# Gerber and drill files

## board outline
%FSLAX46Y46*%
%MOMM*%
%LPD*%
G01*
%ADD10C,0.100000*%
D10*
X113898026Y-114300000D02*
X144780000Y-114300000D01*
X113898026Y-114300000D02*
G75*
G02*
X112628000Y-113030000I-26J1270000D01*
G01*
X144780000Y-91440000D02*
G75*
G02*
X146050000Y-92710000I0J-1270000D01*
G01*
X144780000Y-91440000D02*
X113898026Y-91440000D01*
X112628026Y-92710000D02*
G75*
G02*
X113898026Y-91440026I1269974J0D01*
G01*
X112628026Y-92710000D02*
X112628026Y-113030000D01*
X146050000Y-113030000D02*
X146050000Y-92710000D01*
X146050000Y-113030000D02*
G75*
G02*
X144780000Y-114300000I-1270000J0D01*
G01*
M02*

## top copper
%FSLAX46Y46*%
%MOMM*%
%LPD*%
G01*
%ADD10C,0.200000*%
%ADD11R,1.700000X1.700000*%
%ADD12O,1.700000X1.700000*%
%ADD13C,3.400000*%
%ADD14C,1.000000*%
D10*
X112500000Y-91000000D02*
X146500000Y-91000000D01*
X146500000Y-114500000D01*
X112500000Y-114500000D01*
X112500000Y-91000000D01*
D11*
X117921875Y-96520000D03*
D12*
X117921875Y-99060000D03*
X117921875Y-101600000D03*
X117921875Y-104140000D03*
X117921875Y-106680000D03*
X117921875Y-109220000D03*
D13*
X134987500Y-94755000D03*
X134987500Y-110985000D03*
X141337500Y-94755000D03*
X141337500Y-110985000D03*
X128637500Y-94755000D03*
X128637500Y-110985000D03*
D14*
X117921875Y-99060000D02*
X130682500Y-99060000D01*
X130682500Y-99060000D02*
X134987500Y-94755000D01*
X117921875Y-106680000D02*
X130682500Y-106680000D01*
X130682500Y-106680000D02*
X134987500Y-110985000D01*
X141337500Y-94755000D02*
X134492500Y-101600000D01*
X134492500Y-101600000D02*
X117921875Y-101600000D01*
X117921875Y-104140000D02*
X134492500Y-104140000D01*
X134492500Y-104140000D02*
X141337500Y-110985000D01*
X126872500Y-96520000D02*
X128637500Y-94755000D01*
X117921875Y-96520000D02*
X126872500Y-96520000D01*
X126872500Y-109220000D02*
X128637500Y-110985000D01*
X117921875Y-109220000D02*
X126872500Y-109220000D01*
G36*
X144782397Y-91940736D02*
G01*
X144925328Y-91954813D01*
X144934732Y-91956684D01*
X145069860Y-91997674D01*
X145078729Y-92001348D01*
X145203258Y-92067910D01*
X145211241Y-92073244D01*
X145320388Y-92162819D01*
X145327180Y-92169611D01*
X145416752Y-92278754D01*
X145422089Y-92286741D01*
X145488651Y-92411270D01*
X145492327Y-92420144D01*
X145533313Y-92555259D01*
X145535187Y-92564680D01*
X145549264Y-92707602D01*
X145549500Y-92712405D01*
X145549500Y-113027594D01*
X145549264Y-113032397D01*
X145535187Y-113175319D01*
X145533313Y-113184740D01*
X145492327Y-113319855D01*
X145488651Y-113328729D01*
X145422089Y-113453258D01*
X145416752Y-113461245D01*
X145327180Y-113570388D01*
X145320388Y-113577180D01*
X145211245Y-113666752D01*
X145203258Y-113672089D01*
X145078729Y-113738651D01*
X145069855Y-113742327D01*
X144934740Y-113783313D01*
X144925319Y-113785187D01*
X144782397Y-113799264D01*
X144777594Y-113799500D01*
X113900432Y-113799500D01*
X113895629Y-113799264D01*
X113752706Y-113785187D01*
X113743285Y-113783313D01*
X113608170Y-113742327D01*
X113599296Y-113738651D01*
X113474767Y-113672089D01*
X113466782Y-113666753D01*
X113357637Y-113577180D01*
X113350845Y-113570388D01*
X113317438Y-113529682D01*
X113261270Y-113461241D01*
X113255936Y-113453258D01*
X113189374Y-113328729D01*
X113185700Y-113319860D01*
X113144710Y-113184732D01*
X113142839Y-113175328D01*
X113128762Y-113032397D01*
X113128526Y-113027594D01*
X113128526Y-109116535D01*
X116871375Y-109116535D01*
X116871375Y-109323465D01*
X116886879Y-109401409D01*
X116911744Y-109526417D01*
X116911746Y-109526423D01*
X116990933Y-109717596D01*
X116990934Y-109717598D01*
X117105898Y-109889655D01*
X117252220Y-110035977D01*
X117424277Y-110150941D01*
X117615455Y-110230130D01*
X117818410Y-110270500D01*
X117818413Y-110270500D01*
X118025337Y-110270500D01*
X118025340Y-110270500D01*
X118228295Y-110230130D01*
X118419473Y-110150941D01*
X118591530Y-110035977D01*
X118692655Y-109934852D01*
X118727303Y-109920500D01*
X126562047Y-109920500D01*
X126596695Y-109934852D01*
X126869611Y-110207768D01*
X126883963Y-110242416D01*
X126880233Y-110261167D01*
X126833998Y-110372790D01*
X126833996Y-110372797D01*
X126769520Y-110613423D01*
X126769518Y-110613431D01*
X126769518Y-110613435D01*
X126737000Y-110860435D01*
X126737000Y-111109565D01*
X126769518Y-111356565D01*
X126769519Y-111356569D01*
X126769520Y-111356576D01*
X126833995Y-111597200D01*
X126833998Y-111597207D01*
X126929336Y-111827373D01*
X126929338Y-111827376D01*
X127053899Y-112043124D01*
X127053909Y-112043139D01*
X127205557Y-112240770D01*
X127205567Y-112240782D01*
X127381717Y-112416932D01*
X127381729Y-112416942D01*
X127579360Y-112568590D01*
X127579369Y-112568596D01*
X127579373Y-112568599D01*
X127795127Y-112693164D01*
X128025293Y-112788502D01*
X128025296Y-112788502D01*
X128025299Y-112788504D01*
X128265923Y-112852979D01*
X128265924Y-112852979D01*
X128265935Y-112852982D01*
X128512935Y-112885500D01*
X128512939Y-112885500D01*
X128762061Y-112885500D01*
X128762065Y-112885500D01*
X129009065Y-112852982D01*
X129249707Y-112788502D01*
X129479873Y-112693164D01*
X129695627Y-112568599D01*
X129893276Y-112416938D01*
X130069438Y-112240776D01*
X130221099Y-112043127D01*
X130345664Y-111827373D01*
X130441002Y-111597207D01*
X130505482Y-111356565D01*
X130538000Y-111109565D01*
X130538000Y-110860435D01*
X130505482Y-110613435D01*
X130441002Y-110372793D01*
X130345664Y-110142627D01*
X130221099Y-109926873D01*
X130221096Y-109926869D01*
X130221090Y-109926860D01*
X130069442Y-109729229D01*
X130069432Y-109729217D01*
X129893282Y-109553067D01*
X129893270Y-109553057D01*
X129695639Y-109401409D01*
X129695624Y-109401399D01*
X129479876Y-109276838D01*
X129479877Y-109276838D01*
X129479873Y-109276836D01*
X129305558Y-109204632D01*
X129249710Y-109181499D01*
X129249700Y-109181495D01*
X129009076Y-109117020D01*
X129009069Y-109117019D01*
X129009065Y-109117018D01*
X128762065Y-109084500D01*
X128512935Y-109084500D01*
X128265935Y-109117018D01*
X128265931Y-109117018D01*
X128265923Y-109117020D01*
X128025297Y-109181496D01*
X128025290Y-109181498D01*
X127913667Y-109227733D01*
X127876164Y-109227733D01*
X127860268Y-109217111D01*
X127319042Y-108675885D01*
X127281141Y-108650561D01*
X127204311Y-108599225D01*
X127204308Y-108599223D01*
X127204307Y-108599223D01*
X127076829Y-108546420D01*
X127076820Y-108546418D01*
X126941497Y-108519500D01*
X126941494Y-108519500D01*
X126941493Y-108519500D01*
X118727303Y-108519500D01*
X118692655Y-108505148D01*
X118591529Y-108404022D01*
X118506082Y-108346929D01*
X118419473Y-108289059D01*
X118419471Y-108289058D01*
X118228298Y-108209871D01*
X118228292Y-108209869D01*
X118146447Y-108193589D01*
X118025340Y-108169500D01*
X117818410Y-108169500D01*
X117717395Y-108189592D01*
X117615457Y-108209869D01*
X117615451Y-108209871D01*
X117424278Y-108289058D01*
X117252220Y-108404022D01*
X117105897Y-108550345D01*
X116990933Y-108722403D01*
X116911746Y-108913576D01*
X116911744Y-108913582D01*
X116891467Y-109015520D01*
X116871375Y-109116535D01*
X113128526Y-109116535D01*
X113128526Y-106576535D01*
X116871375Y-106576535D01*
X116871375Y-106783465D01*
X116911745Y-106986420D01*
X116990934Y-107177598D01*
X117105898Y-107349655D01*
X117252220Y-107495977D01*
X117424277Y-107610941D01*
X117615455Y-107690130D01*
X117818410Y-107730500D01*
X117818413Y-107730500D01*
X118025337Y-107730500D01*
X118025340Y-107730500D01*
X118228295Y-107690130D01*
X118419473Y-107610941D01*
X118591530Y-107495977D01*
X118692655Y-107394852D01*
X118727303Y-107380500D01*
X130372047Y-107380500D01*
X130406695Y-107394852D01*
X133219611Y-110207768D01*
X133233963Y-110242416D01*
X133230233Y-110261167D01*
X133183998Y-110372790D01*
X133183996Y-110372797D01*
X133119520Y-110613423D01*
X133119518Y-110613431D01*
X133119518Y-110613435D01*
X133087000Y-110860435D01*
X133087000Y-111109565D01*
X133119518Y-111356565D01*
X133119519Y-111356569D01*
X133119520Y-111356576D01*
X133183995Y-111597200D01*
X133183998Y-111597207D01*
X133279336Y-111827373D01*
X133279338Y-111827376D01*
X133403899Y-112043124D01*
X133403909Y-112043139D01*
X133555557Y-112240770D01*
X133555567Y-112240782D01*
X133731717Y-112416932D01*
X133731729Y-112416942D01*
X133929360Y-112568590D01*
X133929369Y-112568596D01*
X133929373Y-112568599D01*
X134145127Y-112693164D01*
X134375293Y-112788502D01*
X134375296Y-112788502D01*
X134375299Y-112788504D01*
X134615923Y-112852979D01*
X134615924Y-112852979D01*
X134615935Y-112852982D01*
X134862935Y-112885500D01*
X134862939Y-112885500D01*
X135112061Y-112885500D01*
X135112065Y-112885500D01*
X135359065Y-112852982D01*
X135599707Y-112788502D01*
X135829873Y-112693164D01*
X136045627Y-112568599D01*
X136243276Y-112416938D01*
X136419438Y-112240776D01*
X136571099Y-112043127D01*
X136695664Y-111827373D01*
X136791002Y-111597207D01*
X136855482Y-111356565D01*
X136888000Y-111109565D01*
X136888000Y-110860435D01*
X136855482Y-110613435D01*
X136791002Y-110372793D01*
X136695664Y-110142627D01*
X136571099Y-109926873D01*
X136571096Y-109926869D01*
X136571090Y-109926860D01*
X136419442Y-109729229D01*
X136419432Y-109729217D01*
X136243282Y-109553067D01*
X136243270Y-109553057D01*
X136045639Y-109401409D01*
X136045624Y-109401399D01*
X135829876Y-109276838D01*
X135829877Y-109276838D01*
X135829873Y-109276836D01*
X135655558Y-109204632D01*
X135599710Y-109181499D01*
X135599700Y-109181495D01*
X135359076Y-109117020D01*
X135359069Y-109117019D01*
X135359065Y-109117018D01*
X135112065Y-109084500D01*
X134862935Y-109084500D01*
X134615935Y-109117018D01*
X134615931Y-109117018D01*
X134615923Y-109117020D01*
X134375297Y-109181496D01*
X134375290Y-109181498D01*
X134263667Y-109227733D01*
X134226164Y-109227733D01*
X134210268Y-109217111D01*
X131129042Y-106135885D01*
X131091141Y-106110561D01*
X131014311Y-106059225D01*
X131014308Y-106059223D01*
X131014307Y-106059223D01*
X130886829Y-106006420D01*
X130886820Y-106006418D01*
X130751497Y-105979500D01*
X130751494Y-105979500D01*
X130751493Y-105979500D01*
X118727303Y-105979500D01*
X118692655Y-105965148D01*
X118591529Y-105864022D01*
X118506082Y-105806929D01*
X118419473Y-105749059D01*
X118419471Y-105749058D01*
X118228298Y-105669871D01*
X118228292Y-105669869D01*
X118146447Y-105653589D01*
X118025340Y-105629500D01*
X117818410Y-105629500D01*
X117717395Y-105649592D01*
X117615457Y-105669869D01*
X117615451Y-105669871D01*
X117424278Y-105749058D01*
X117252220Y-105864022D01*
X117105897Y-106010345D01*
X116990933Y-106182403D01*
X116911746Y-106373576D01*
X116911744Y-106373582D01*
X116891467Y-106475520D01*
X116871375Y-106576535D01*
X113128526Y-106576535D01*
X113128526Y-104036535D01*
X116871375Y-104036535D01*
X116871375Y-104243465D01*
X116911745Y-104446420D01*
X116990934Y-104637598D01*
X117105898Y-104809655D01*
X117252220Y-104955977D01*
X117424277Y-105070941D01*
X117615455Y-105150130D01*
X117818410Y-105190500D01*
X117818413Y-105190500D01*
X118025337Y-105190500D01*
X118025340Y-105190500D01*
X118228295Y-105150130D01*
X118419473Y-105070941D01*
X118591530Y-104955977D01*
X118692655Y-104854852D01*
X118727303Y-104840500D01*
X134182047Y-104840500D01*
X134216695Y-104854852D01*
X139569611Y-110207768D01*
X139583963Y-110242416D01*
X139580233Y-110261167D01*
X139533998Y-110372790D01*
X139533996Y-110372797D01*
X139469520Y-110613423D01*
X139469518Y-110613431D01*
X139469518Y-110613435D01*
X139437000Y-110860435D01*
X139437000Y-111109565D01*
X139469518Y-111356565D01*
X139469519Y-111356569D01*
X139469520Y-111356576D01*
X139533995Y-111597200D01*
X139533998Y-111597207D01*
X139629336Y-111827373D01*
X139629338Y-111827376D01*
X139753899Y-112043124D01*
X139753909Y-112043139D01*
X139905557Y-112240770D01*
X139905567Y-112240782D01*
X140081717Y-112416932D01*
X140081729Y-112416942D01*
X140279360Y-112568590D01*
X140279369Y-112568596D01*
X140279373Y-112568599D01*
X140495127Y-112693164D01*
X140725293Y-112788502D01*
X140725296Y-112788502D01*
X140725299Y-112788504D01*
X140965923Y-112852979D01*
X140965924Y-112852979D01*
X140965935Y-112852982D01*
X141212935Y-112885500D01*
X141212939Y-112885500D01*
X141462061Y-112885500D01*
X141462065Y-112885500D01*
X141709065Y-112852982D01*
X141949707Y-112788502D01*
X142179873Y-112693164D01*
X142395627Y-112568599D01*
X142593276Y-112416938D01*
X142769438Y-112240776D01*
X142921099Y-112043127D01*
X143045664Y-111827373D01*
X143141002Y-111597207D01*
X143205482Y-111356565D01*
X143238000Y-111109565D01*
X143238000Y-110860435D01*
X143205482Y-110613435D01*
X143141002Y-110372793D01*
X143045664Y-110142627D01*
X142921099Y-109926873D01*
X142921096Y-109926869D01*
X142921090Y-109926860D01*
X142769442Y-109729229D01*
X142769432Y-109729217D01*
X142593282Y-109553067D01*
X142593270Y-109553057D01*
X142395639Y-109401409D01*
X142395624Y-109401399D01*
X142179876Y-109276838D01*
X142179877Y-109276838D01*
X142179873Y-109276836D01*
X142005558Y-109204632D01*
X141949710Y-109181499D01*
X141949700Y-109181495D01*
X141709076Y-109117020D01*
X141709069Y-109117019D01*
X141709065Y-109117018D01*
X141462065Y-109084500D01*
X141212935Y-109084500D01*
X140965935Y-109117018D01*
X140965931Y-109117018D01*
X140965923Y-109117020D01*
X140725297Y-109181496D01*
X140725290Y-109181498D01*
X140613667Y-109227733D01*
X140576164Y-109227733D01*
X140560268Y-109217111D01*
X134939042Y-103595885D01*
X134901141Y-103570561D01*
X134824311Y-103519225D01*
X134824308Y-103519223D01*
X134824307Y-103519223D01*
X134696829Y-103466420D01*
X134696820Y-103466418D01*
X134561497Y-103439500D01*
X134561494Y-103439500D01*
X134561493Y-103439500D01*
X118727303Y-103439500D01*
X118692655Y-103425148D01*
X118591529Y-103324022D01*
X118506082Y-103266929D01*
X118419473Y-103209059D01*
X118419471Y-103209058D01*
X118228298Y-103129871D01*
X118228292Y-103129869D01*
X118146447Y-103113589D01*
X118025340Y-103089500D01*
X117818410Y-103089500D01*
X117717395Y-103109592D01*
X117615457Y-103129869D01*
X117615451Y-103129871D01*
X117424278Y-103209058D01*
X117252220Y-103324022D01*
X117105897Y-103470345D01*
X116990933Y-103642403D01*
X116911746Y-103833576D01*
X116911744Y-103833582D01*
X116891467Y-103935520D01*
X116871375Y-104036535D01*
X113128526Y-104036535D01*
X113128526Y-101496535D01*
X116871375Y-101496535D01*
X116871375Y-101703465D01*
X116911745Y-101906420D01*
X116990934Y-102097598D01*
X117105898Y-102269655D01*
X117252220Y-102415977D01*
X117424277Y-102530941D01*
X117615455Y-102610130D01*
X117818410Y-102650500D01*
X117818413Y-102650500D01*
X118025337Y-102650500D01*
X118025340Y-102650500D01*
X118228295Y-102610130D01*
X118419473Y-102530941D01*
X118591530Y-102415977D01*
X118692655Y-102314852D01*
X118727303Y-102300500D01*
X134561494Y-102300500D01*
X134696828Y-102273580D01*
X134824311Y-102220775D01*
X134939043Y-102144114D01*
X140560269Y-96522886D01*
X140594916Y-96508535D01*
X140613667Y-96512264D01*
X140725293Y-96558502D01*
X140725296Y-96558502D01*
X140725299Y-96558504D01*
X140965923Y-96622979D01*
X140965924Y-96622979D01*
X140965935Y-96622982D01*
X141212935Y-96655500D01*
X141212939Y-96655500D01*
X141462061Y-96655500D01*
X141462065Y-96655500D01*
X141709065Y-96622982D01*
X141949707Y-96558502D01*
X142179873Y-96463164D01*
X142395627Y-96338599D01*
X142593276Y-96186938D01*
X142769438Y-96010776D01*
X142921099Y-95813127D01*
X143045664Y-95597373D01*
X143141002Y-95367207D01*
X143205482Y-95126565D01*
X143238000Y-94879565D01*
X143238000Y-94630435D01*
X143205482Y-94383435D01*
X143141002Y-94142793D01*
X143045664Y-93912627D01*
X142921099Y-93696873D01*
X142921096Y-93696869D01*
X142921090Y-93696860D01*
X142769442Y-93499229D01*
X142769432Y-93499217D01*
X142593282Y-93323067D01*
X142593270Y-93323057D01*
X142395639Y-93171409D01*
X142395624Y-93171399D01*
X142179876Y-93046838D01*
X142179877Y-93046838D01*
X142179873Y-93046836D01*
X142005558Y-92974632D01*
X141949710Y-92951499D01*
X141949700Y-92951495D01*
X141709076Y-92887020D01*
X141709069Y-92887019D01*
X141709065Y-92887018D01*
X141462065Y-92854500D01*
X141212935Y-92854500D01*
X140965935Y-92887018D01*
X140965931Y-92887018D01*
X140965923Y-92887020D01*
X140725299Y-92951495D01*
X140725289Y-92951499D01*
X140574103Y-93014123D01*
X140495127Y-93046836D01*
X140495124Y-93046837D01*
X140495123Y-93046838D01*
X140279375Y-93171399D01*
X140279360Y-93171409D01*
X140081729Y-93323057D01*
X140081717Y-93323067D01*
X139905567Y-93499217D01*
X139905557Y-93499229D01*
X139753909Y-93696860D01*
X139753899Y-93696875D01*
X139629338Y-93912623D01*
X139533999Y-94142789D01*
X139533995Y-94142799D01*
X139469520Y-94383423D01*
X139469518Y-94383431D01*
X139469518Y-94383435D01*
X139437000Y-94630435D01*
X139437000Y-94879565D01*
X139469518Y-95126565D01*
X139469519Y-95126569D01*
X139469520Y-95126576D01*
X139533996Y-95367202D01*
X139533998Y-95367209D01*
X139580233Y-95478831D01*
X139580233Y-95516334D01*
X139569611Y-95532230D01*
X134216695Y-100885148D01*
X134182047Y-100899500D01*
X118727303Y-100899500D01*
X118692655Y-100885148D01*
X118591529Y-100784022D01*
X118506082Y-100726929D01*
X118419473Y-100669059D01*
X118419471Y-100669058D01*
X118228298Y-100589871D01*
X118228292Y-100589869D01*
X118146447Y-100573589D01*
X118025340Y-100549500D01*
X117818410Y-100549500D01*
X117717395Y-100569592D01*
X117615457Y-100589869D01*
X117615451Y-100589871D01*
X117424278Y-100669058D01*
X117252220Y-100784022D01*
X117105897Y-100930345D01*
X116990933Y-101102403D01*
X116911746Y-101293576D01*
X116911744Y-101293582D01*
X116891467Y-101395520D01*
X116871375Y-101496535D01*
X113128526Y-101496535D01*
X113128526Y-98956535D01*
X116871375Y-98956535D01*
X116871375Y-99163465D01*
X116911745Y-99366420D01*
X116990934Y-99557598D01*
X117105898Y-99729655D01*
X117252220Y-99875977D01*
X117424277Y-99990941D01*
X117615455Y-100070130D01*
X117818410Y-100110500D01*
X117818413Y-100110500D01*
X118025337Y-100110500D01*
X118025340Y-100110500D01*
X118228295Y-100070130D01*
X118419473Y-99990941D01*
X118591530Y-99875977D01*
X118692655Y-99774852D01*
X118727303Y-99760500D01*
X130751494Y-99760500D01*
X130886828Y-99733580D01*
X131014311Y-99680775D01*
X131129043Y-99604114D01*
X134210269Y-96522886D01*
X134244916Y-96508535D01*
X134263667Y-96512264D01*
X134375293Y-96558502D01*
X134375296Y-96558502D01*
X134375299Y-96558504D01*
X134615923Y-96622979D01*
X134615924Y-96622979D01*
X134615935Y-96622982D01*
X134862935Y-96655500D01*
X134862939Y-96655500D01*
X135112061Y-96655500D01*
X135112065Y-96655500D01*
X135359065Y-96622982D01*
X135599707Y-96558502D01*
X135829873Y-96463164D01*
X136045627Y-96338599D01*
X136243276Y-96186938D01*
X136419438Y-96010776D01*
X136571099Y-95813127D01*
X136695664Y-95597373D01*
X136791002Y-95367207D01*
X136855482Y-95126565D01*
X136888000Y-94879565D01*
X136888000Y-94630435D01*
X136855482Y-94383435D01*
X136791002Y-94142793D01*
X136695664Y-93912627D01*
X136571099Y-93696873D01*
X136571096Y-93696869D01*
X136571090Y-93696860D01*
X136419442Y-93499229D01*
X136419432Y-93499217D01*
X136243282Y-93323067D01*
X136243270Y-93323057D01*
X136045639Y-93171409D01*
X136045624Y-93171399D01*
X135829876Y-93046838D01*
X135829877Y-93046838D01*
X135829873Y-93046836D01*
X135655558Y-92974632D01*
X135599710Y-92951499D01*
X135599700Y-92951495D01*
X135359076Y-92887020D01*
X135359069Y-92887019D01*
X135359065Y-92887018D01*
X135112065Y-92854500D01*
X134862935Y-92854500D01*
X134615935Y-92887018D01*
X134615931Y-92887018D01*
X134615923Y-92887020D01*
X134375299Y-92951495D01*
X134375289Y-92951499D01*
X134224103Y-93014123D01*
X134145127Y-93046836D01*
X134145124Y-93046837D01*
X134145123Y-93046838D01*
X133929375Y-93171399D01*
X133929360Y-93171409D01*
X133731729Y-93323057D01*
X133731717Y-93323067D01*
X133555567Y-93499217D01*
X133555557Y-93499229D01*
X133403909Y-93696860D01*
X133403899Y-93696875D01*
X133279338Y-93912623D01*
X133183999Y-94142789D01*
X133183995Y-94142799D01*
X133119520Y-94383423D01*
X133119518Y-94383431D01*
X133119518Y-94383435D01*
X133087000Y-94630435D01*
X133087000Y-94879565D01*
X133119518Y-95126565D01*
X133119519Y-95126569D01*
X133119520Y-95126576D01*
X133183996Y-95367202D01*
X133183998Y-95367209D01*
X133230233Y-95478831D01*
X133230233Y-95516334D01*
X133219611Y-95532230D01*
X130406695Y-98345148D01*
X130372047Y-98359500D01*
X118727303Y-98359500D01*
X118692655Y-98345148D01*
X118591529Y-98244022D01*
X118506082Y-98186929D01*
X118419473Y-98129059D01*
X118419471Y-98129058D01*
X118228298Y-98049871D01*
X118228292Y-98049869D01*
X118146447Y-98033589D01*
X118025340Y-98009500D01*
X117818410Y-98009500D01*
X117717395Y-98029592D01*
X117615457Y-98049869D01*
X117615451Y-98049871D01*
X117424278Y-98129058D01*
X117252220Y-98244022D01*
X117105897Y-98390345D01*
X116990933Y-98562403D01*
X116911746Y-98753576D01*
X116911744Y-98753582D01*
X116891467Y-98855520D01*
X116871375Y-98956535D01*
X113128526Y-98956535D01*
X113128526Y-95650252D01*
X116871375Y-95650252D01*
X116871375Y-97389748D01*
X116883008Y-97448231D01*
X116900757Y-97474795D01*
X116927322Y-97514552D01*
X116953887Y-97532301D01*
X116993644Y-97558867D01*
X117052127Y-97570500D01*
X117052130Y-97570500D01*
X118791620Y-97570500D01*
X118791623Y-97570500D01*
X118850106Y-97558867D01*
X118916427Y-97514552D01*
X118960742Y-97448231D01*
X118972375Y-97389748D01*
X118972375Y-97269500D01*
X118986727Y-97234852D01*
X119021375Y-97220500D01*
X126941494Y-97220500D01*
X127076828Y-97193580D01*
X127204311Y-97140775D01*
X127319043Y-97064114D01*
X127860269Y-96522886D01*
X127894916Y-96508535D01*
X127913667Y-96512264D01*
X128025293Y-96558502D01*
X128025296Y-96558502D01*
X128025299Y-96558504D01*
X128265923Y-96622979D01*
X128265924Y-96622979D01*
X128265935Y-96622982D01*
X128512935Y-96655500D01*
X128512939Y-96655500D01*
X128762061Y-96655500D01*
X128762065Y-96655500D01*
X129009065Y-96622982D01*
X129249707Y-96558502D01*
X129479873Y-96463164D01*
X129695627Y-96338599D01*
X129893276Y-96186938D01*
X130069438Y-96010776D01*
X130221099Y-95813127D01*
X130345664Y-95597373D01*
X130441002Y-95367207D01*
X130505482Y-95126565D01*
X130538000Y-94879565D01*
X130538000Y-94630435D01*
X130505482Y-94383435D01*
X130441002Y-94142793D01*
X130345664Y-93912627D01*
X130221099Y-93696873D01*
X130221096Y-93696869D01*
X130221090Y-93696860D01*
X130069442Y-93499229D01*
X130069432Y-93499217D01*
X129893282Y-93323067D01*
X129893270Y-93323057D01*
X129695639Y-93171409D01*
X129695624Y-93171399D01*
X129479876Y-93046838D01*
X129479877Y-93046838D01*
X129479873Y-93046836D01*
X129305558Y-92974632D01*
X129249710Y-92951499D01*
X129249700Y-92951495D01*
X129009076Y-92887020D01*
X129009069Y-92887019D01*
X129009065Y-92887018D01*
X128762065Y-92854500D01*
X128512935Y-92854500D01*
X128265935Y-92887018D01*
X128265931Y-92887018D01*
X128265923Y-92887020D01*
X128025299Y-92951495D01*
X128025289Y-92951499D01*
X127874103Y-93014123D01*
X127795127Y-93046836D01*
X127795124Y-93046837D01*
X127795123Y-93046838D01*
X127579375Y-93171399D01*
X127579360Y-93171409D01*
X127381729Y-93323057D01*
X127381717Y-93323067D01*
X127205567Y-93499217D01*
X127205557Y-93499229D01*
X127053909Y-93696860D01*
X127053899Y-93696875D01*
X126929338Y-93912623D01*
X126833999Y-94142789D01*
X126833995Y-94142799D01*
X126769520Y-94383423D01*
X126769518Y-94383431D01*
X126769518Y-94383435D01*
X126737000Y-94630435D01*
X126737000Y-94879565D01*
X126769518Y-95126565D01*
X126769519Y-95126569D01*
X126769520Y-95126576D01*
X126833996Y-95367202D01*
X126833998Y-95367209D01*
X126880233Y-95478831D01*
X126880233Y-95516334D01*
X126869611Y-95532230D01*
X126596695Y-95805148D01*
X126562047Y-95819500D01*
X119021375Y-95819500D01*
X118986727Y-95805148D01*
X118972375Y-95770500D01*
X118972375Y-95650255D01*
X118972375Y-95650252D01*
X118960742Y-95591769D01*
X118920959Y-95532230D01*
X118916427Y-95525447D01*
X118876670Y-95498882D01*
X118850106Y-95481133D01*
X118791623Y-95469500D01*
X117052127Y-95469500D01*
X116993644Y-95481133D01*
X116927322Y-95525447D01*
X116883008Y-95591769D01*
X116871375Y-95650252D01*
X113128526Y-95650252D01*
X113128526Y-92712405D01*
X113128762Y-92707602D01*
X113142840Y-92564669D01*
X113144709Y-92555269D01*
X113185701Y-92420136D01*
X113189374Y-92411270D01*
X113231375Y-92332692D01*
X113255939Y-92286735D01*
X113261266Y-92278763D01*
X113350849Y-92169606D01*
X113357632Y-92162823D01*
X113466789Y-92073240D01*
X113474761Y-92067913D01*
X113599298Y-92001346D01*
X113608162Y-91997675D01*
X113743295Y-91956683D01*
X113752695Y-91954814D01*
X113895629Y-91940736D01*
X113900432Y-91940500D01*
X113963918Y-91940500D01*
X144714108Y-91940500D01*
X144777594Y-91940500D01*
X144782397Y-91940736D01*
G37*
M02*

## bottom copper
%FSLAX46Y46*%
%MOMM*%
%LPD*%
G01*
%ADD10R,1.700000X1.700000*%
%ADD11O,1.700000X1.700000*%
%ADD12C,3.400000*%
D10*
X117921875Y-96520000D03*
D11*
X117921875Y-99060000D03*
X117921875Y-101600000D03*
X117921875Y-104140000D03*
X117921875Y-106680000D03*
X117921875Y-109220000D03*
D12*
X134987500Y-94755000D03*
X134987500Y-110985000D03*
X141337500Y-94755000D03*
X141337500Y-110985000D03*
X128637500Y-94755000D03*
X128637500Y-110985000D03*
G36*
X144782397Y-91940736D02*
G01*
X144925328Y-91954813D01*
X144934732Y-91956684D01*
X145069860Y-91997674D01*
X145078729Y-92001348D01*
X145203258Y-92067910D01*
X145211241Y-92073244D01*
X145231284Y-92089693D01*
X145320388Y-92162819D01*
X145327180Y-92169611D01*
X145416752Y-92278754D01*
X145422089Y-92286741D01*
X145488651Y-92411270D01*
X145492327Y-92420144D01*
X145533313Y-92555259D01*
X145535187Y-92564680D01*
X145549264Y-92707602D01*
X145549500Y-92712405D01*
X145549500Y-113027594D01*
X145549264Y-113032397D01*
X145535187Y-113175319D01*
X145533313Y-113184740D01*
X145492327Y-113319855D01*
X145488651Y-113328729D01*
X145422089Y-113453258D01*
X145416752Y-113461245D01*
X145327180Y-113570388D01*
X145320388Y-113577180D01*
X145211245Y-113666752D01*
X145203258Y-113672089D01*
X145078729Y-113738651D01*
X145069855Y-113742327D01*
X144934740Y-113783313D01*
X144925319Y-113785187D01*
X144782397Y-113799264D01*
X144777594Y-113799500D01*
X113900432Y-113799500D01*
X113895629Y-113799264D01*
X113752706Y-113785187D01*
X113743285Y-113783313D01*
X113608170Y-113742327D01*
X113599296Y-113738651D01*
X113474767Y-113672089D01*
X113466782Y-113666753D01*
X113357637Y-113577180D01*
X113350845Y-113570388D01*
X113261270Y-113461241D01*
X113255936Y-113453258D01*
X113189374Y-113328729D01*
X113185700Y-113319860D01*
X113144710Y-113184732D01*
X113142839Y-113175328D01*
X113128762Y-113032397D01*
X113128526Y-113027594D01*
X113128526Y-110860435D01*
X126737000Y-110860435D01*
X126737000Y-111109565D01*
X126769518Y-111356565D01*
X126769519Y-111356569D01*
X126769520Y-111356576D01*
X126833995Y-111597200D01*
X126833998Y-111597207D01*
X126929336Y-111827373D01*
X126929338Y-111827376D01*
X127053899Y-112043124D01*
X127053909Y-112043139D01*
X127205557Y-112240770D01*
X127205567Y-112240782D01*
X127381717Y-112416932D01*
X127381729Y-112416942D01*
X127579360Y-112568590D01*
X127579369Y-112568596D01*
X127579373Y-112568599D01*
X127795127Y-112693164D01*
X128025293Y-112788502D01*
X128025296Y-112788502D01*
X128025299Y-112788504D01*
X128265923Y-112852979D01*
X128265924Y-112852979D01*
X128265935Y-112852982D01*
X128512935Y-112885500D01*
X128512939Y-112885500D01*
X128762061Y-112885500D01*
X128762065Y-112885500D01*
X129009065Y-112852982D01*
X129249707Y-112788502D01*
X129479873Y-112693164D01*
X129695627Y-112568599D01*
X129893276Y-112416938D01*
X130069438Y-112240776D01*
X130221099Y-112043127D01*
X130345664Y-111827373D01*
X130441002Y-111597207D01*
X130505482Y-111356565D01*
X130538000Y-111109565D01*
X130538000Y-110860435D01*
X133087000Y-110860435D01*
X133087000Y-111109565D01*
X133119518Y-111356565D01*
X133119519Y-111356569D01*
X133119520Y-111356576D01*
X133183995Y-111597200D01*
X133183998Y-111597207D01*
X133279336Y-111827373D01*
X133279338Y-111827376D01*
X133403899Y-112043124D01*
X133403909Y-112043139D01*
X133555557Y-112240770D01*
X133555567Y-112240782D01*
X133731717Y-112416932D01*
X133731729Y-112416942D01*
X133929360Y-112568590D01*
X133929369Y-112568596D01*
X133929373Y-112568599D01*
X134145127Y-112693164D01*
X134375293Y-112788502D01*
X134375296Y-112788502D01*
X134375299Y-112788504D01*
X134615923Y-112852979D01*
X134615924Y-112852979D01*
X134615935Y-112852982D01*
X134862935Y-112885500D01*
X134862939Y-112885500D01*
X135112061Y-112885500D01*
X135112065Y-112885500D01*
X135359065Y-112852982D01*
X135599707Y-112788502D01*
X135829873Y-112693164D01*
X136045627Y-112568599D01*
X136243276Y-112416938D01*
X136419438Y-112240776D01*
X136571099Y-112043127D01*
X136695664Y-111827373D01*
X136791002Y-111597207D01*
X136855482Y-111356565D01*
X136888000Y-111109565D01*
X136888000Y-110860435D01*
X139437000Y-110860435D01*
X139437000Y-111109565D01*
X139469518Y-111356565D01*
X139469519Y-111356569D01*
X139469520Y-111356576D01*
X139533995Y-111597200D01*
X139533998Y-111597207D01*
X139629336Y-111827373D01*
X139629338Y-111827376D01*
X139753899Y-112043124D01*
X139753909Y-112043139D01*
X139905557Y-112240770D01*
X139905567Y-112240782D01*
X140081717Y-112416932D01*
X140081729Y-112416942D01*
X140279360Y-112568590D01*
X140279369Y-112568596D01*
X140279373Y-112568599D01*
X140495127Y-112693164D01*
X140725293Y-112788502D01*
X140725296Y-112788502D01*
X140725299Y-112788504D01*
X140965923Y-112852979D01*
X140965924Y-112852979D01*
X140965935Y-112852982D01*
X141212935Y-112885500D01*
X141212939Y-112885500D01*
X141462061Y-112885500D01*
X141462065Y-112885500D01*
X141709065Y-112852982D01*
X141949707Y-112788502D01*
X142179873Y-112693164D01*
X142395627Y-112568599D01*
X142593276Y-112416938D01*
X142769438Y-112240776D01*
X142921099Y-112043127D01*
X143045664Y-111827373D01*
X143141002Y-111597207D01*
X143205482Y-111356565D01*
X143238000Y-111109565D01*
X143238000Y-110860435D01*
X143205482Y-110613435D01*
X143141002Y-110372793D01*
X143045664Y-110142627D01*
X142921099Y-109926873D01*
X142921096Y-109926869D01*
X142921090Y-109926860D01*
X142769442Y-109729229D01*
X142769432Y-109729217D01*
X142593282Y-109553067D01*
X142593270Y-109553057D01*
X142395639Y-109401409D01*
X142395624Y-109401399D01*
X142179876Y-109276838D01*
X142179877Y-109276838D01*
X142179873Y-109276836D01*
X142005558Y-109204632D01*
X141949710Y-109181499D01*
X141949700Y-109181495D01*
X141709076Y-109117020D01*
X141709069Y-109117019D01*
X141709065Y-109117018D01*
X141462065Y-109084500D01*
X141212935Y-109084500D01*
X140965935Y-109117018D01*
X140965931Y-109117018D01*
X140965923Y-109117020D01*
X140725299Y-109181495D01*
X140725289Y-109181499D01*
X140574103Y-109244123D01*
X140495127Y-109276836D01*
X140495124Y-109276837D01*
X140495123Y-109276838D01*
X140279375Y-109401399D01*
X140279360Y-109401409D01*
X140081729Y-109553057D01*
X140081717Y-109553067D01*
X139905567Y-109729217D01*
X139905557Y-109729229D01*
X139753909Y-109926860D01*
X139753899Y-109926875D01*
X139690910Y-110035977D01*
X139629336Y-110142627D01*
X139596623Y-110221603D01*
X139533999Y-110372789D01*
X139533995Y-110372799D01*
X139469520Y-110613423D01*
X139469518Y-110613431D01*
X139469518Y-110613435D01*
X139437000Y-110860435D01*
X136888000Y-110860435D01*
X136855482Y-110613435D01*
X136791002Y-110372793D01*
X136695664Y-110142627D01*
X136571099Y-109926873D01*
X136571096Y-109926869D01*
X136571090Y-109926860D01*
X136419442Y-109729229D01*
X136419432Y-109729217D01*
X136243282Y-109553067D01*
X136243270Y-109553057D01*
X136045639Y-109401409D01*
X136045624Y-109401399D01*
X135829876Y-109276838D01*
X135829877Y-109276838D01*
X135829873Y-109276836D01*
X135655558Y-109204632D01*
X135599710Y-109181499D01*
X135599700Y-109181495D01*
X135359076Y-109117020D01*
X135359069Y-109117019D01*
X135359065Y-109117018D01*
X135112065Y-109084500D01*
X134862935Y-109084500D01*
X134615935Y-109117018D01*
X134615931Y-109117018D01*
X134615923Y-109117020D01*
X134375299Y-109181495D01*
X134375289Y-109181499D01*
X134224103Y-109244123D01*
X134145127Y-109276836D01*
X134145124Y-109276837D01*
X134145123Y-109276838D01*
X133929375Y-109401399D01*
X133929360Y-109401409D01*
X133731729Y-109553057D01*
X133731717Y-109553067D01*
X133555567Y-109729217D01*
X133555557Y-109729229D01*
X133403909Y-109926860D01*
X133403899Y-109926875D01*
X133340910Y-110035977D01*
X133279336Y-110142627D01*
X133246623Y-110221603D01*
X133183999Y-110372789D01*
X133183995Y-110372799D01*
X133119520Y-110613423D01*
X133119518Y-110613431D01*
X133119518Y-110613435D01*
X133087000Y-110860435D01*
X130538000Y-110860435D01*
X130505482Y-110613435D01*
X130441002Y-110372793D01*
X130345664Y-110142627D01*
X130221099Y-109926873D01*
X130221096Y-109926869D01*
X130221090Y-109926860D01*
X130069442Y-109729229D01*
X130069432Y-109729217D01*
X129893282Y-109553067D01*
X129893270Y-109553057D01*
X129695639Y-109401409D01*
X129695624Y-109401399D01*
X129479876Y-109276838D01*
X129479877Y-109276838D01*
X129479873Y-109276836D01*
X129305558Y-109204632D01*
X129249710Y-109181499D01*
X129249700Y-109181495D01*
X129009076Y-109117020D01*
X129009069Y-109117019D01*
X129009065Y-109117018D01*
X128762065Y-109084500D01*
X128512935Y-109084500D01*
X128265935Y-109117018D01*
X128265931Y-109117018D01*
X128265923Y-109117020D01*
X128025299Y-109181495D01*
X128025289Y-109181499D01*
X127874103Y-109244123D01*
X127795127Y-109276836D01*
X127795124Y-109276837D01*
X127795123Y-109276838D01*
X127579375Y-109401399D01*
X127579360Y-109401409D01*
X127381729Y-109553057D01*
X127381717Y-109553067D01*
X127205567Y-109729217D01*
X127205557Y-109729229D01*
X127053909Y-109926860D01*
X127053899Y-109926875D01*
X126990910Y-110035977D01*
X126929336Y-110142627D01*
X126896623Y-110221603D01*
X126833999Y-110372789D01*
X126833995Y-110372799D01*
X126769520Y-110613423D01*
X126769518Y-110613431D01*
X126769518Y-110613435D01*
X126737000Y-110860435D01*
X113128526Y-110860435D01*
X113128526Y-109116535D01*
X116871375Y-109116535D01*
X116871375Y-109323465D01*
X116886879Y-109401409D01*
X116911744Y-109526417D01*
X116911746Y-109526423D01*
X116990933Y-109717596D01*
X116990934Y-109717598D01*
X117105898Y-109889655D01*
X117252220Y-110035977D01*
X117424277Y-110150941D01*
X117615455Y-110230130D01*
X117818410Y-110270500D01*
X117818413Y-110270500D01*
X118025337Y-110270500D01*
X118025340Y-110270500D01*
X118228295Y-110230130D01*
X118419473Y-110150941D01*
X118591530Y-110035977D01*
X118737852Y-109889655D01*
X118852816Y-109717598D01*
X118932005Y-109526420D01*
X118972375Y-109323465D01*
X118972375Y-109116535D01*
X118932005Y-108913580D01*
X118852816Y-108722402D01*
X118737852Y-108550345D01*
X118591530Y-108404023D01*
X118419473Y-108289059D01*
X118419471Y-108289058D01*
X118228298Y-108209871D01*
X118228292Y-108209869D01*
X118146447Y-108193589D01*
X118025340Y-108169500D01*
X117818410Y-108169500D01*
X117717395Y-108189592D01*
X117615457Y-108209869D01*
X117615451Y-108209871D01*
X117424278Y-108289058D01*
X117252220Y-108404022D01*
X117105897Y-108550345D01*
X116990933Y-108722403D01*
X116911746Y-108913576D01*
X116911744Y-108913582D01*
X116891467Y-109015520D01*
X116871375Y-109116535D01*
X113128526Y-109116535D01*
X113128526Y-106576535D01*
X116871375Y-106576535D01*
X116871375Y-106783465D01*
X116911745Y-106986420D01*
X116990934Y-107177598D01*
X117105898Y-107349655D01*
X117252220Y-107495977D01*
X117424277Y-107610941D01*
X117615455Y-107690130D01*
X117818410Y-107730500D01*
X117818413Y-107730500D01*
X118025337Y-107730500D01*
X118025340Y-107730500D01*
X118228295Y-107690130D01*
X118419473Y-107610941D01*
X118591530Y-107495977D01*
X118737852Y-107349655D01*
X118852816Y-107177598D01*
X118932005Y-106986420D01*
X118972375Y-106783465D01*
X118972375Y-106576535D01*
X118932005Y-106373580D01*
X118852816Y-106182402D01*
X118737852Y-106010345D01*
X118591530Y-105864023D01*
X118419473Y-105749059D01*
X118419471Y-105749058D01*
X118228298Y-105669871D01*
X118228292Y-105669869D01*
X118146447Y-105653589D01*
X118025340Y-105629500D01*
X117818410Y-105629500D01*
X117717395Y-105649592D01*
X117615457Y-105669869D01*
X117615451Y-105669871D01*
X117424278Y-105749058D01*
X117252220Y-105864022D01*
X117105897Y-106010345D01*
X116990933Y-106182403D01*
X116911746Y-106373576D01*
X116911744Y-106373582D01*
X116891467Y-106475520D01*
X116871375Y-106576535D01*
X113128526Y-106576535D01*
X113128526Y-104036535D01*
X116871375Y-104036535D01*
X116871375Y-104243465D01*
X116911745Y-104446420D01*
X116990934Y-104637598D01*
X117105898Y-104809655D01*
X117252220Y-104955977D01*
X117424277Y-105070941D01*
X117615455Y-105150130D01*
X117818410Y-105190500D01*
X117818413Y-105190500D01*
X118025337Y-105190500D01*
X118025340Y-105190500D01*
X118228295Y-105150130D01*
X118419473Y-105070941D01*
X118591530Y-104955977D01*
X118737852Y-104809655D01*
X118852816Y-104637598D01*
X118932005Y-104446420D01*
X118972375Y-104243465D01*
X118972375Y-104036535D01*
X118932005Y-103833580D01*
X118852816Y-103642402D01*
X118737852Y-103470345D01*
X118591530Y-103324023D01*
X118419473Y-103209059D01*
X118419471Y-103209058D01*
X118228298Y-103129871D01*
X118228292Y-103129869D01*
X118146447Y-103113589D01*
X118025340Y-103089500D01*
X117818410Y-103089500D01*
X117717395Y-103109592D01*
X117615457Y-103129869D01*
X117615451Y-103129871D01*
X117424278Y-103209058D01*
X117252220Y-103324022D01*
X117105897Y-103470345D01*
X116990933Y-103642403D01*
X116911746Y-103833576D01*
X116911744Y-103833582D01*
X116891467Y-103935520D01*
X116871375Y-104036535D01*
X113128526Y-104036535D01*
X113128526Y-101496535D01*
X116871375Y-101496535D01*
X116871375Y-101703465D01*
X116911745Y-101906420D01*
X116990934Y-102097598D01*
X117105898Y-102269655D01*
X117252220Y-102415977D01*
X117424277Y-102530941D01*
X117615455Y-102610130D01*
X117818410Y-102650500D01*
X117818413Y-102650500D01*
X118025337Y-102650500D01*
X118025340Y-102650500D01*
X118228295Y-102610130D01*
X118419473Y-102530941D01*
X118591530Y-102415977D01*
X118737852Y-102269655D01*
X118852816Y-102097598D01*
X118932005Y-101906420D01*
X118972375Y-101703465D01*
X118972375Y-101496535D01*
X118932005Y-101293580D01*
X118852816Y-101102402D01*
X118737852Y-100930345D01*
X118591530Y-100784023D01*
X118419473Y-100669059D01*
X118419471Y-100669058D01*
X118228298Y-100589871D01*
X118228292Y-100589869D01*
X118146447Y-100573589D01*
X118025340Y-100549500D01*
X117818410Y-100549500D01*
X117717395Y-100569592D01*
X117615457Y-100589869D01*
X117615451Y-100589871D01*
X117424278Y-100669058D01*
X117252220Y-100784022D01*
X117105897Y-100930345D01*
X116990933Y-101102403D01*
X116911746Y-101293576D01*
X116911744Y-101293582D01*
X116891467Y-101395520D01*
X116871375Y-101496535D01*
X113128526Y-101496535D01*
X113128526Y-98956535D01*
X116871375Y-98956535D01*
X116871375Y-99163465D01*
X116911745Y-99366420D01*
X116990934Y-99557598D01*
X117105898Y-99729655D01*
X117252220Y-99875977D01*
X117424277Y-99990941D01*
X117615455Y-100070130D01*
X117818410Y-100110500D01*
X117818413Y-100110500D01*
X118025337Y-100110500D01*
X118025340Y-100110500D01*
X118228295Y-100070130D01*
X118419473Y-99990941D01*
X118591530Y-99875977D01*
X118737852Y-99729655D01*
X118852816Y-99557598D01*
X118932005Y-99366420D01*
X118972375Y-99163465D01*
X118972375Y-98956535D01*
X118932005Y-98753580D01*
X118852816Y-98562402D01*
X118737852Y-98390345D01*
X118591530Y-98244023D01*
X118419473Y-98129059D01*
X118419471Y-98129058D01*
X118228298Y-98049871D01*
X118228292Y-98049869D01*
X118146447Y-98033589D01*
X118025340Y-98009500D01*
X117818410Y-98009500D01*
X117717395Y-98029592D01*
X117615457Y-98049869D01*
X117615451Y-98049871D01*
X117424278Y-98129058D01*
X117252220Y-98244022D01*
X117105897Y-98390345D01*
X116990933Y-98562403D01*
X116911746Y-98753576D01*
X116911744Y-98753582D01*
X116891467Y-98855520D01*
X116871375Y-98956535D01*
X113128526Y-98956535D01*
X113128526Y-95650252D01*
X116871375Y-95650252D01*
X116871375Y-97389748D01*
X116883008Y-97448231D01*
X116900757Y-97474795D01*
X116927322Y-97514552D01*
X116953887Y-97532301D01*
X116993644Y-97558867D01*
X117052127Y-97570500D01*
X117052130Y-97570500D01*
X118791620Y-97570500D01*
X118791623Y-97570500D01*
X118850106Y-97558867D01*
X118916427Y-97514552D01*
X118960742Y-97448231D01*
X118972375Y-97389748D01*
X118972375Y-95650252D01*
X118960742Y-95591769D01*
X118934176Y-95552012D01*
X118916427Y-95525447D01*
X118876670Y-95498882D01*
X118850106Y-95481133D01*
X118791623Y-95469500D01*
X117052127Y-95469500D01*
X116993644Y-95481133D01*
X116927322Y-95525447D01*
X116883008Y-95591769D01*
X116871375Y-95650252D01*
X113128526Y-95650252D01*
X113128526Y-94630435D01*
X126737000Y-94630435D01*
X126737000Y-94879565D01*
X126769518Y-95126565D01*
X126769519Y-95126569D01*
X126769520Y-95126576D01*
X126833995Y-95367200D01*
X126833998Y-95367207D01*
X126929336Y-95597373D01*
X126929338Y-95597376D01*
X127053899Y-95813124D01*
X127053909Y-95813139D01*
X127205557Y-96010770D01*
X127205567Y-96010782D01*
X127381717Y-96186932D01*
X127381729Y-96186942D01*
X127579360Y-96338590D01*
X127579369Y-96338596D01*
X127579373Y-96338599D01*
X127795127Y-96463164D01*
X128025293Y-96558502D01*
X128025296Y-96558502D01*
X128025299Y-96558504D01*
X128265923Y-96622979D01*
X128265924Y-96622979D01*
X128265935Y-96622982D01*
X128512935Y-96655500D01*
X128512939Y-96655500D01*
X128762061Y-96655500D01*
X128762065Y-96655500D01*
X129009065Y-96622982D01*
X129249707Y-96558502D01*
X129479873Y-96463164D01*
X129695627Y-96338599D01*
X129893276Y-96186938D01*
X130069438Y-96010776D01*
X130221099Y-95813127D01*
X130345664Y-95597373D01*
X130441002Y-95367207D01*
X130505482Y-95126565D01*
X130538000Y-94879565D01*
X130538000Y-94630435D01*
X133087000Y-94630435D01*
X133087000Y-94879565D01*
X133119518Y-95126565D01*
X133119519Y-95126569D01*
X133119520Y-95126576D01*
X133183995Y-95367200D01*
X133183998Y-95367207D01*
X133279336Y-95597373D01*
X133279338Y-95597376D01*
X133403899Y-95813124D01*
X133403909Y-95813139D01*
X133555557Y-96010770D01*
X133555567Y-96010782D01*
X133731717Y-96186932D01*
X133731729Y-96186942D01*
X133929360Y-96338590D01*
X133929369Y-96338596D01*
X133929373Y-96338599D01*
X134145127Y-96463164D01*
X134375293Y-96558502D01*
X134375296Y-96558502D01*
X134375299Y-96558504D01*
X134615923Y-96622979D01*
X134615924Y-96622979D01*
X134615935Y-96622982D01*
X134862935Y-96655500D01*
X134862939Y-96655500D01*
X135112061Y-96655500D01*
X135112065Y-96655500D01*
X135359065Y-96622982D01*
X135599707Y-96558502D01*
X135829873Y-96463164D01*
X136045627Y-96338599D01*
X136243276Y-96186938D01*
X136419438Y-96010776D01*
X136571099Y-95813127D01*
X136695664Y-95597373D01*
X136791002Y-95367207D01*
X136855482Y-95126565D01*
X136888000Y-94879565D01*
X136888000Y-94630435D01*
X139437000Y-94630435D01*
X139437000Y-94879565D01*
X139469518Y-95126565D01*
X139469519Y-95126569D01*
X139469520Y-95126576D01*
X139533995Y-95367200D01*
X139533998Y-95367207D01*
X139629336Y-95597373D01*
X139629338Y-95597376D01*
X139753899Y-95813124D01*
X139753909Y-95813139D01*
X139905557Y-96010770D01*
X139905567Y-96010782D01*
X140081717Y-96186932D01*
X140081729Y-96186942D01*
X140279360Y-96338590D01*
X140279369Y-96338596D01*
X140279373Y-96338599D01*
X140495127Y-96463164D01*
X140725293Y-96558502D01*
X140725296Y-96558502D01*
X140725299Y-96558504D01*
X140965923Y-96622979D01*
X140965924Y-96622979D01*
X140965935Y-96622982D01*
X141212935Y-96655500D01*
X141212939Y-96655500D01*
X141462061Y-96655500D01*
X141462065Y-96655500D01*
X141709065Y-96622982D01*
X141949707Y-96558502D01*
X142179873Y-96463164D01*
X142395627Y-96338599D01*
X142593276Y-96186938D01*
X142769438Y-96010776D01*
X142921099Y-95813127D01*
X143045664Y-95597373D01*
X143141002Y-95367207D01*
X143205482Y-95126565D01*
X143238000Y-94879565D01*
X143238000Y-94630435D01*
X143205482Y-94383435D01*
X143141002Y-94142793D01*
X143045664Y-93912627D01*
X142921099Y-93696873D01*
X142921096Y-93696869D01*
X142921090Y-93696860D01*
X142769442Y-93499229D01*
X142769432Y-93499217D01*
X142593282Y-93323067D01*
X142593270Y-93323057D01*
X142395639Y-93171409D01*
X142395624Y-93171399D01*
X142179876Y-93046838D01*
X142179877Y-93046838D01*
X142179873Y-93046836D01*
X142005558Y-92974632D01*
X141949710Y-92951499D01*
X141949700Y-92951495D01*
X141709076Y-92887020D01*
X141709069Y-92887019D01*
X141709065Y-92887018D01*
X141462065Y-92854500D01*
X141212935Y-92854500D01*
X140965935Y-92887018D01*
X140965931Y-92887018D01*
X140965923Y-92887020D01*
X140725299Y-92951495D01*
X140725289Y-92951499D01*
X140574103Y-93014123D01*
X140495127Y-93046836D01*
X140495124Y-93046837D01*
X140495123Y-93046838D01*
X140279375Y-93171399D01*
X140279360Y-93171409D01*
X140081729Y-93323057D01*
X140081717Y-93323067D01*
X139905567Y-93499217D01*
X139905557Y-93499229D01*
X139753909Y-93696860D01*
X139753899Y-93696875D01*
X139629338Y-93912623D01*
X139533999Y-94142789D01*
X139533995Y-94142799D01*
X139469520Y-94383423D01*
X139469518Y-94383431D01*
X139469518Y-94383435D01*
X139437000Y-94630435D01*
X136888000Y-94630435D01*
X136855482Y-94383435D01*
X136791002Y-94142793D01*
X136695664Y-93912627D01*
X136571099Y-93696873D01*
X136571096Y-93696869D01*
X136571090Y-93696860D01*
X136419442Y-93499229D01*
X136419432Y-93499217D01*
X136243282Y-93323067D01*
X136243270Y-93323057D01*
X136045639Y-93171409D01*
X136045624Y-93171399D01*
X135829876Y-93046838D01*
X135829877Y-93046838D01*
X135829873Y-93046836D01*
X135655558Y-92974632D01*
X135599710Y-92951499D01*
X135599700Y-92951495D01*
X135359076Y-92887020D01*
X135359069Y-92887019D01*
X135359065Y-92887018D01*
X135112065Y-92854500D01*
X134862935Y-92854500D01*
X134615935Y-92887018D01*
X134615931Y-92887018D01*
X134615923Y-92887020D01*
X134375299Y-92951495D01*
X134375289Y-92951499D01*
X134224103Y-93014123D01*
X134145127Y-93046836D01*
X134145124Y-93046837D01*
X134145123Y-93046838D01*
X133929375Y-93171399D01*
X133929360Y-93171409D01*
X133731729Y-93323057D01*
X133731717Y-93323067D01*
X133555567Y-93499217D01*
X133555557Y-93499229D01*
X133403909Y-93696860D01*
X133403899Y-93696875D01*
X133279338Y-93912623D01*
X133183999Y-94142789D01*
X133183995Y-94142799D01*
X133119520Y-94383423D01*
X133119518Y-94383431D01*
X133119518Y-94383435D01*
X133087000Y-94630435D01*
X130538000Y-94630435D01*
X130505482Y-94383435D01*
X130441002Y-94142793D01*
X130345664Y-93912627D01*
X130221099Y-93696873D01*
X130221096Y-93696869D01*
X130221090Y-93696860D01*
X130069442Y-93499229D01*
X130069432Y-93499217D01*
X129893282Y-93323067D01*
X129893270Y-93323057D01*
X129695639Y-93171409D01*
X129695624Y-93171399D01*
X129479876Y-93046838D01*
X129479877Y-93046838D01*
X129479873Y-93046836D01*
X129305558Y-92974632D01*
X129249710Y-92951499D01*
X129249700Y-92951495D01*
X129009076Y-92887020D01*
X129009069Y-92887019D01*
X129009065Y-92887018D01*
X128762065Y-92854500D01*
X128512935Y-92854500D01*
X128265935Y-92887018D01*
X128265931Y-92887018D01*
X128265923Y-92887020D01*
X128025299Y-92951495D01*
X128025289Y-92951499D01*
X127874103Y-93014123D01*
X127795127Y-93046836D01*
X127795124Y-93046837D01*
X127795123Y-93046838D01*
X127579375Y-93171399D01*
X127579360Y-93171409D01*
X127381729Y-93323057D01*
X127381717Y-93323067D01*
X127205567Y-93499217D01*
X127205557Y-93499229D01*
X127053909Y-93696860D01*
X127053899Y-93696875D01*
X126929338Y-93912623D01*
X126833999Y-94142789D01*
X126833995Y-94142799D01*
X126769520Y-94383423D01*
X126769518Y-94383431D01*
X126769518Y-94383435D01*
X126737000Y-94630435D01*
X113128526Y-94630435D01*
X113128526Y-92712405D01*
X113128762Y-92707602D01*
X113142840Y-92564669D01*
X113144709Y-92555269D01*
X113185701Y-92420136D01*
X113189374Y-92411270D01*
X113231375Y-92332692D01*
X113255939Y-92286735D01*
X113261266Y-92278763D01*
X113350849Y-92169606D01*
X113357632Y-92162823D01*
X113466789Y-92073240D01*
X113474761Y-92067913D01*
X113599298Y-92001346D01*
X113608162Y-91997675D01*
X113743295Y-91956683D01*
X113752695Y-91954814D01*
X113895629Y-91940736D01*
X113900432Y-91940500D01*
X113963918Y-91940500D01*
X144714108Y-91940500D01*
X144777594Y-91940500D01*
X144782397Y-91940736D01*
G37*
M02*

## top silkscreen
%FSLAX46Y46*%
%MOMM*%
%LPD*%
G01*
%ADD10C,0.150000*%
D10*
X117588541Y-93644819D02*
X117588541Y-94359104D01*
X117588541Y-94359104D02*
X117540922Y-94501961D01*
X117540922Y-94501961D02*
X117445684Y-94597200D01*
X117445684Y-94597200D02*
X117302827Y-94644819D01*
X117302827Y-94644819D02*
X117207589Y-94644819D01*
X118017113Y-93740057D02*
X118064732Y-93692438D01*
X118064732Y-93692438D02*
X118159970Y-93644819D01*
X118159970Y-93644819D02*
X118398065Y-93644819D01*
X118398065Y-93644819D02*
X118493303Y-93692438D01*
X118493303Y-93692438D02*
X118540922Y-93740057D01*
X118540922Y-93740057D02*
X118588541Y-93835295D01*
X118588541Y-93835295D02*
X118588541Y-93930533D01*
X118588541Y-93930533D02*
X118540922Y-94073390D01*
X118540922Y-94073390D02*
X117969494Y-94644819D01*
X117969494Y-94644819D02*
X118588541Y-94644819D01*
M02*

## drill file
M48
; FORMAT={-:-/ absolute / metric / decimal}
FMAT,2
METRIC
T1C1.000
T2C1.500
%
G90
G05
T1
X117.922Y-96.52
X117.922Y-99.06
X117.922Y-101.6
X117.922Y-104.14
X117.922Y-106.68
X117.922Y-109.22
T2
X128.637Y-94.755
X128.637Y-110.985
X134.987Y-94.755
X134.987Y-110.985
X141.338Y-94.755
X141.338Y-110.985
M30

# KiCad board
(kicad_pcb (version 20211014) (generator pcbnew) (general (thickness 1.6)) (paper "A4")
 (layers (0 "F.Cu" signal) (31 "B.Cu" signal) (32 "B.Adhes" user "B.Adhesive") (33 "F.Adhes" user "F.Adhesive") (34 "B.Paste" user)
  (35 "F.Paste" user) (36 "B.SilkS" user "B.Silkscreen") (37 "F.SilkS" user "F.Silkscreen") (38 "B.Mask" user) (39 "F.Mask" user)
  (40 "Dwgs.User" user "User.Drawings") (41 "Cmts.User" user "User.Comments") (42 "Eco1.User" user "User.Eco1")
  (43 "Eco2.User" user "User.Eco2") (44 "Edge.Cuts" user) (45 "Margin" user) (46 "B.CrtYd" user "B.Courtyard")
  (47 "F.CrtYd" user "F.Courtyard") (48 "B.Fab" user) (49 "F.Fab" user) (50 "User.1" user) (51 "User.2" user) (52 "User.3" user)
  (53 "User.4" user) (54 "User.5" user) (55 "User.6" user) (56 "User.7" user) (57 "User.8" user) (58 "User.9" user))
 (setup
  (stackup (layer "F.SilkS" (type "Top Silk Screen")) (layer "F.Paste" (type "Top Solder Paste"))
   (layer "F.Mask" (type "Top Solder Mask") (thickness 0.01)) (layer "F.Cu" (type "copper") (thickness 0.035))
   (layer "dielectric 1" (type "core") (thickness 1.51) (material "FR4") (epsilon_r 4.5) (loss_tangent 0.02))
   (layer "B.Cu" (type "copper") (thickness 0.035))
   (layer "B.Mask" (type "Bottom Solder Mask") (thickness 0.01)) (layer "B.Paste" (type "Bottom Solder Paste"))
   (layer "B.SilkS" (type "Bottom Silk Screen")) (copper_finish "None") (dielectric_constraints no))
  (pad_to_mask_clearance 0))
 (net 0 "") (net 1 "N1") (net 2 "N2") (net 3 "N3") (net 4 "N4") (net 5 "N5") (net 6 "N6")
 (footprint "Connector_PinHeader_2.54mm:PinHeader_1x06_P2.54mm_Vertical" (layer "F.Cu") (at 117.921875 96.52)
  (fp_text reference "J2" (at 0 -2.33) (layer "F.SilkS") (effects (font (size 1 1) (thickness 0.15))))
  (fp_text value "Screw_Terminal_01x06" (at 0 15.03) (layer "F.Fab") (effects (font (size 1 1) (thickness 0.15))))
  (pad "1" thru_hole rect (at 0 0) (size 1.7 1.7) (drill 1) (layers *.Cu *.Mask) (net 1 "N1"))
  (pad "2" thru_hole oval (at 0 2.54) (size 1.7 1.7) (drill 1) (layers *.Cu *.Mask) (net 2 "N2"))
  (pad "3" thru_hole oval (at 0 5.08) (size 1.7 1.7) (drill 1) (layers *.Cu *.Mask) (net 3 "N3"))
  (pad "4" thru_hole oval (at 0 7.62) (size 1.7 1.7) (drill 1) (layers *.Cu *.Mask) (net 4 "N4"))
  (pad "5" thru_hole oval (at 0 10.16) (size 1.7 1.7) (drill 1) (layers *.Cu *.Mask) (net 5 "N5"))
  (pad "6" thru_hole oval (at 0 12.7) (size 1.7 1.7) (drill 1) (layers *.Cu *.Mask) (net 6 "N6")))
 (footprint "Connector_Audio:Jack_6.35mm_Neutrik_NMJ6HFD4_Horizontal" (layer "F.Cu") (at 128.6375 94.755)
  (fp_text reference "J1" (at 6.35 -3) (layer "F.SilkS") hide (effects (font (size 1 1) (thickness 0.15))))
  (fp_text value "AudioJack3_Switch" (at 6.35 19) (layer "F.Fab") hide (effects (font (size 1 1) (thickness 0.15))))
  (pad "R" thru_hole circle (at 6.35 0) (size 3.4 3.4) (drill 1.5) (layers *.Cu *.Mask) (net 2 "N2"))
  (pad "RN" thru_hole circle (at 6.35 16.23) (size 3.4 3.4) (drill 1.5) (layers *.Cu *.Mask) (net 5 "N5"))
  (pad "S" thru_hole circle (at 12.7 0) (size 3.4 3.4) (drill 1.5) (layers *.Cu *.Mask) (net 3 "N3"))
  (pad "SN" thru_hole circle (at 12.7 16.23) (size 3.4 3.4) (drill 1.5) (layers *.Cu *.Mask) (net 4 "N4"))
  (pad "T" thru_hole circle (at 0 0) (size 3.4 3.4) (drill 1.5) (layers *.Cu *.Mask) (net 1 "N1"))
  (pad "TN" thru_hole circle (at 0 16.23) (size 3.4 3.4) (drill 1.5) (layers *.Cu *.Mask) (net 6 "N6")))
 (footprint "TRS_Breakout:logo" (layer "B.Cu") (at 135 102.87 180)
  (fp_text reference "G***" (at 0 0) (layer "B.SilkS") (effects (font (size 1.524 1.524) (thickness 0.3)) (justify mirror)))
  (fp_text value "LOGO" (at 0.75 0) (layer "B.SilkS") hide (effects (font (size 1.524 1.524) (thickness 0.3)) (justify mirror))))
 (gr_rect (start 112.5 91) (end 146.5 114.5) (layer "F.Cu") (width 0.2) (fill none))
 (gr_line (start 113.898026 114.3) (end 144.78 114.3) (layer "Edge.Cuts") (width 0.1))
 (gr_arc (start 113.898026 114.3) (mid 113 113.928026) (end 112.628026 113.03) (layer "Edge.Cuts") (width 0.1))
 (gr_arc (start 144.78 91.44) (mid 145.678026 91.811974) (end 146.05 92.71) (layer "Edge.Cuts") (width 0.1))
 (gr_line (start 144.78 91.44) (end 113.898026 91.44) (layer "Edge.Cuts") (width 0.1))
 (gr_arc (start 112.628026 92.71) (mid 113 91.811974) (end 113.898026 91.44) (layer "Edge.Cuts") (width 0.1))
 (gr_line (start 112.628026 92.71) (end 112.628026 113.03) (layer "Edge.Cuts") (width 0.1))
 (gr_line (start 146.05 113.03) (end 146.05 92.71) (layer "Edge.Cuts") (width 0.1))
 (gr_arc (start 146.05 113.03) (mid 145.678026 113.928026) (end 144.78 114.3) (layer "Edge.Cuts") (width 0.1))
 (segment (start 117.921875 99.06) (end 130.6825 99.06) (width 1) (layer "F.Cu") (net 2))
 (segment (start 130.6825 99.06) (end 134.9875 94.755) (width 1) (layer "F.Cu") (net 2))
 (segment (start 117.921875 106.68) (end 130.6825 106.68) (width 1) (layer "F.Cu") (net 5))
 (segment (start 130.6825 106.68) (end 134.9875 110.985) (width 1) (layer "F.Cu") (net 5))
 (segment (start 141.3375 94.755) (end 134.4925 101.6) (width 1) (layer "F.Cu") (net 3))
 (segment (start 134.4925 101.6) (end 117.921875 101.6) (width 1) (layer "F.Cu") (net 3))
 (segment (start 117.921875 104.14) (end 134.4925 104.14) (width 1) (layer "F.Cu") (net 4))
 (segment (start 134.4925 104.14) (end 141.3375 110.985) (width 1) (layer "F.Cu") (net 4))
 (segment (start 126.8725 96.52) (end 128.6375 94.755) (width 1) (layer "F.Cu") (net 1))
 (segment (start 117.921875 96.52) (end 126.8725 96.52) (width 1) (layer "F.Cu") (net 1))
 (segment (start 126.8725 109.22) (end 128.6375 110.985) (width 1) (layer "F.Cu") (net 6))
 (segment (start 117.921875 109.22) (end 126.8725 109.22) (width 1) (layer "F.Cu") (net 6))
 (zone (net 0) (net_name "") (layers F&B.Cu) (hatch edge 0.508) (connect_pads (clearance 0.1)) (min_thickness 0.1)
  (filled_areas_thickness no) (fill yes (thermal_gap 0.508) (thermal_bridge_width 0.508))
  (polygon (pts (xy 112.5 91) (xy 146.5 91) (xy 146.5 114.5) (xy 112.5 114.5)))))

